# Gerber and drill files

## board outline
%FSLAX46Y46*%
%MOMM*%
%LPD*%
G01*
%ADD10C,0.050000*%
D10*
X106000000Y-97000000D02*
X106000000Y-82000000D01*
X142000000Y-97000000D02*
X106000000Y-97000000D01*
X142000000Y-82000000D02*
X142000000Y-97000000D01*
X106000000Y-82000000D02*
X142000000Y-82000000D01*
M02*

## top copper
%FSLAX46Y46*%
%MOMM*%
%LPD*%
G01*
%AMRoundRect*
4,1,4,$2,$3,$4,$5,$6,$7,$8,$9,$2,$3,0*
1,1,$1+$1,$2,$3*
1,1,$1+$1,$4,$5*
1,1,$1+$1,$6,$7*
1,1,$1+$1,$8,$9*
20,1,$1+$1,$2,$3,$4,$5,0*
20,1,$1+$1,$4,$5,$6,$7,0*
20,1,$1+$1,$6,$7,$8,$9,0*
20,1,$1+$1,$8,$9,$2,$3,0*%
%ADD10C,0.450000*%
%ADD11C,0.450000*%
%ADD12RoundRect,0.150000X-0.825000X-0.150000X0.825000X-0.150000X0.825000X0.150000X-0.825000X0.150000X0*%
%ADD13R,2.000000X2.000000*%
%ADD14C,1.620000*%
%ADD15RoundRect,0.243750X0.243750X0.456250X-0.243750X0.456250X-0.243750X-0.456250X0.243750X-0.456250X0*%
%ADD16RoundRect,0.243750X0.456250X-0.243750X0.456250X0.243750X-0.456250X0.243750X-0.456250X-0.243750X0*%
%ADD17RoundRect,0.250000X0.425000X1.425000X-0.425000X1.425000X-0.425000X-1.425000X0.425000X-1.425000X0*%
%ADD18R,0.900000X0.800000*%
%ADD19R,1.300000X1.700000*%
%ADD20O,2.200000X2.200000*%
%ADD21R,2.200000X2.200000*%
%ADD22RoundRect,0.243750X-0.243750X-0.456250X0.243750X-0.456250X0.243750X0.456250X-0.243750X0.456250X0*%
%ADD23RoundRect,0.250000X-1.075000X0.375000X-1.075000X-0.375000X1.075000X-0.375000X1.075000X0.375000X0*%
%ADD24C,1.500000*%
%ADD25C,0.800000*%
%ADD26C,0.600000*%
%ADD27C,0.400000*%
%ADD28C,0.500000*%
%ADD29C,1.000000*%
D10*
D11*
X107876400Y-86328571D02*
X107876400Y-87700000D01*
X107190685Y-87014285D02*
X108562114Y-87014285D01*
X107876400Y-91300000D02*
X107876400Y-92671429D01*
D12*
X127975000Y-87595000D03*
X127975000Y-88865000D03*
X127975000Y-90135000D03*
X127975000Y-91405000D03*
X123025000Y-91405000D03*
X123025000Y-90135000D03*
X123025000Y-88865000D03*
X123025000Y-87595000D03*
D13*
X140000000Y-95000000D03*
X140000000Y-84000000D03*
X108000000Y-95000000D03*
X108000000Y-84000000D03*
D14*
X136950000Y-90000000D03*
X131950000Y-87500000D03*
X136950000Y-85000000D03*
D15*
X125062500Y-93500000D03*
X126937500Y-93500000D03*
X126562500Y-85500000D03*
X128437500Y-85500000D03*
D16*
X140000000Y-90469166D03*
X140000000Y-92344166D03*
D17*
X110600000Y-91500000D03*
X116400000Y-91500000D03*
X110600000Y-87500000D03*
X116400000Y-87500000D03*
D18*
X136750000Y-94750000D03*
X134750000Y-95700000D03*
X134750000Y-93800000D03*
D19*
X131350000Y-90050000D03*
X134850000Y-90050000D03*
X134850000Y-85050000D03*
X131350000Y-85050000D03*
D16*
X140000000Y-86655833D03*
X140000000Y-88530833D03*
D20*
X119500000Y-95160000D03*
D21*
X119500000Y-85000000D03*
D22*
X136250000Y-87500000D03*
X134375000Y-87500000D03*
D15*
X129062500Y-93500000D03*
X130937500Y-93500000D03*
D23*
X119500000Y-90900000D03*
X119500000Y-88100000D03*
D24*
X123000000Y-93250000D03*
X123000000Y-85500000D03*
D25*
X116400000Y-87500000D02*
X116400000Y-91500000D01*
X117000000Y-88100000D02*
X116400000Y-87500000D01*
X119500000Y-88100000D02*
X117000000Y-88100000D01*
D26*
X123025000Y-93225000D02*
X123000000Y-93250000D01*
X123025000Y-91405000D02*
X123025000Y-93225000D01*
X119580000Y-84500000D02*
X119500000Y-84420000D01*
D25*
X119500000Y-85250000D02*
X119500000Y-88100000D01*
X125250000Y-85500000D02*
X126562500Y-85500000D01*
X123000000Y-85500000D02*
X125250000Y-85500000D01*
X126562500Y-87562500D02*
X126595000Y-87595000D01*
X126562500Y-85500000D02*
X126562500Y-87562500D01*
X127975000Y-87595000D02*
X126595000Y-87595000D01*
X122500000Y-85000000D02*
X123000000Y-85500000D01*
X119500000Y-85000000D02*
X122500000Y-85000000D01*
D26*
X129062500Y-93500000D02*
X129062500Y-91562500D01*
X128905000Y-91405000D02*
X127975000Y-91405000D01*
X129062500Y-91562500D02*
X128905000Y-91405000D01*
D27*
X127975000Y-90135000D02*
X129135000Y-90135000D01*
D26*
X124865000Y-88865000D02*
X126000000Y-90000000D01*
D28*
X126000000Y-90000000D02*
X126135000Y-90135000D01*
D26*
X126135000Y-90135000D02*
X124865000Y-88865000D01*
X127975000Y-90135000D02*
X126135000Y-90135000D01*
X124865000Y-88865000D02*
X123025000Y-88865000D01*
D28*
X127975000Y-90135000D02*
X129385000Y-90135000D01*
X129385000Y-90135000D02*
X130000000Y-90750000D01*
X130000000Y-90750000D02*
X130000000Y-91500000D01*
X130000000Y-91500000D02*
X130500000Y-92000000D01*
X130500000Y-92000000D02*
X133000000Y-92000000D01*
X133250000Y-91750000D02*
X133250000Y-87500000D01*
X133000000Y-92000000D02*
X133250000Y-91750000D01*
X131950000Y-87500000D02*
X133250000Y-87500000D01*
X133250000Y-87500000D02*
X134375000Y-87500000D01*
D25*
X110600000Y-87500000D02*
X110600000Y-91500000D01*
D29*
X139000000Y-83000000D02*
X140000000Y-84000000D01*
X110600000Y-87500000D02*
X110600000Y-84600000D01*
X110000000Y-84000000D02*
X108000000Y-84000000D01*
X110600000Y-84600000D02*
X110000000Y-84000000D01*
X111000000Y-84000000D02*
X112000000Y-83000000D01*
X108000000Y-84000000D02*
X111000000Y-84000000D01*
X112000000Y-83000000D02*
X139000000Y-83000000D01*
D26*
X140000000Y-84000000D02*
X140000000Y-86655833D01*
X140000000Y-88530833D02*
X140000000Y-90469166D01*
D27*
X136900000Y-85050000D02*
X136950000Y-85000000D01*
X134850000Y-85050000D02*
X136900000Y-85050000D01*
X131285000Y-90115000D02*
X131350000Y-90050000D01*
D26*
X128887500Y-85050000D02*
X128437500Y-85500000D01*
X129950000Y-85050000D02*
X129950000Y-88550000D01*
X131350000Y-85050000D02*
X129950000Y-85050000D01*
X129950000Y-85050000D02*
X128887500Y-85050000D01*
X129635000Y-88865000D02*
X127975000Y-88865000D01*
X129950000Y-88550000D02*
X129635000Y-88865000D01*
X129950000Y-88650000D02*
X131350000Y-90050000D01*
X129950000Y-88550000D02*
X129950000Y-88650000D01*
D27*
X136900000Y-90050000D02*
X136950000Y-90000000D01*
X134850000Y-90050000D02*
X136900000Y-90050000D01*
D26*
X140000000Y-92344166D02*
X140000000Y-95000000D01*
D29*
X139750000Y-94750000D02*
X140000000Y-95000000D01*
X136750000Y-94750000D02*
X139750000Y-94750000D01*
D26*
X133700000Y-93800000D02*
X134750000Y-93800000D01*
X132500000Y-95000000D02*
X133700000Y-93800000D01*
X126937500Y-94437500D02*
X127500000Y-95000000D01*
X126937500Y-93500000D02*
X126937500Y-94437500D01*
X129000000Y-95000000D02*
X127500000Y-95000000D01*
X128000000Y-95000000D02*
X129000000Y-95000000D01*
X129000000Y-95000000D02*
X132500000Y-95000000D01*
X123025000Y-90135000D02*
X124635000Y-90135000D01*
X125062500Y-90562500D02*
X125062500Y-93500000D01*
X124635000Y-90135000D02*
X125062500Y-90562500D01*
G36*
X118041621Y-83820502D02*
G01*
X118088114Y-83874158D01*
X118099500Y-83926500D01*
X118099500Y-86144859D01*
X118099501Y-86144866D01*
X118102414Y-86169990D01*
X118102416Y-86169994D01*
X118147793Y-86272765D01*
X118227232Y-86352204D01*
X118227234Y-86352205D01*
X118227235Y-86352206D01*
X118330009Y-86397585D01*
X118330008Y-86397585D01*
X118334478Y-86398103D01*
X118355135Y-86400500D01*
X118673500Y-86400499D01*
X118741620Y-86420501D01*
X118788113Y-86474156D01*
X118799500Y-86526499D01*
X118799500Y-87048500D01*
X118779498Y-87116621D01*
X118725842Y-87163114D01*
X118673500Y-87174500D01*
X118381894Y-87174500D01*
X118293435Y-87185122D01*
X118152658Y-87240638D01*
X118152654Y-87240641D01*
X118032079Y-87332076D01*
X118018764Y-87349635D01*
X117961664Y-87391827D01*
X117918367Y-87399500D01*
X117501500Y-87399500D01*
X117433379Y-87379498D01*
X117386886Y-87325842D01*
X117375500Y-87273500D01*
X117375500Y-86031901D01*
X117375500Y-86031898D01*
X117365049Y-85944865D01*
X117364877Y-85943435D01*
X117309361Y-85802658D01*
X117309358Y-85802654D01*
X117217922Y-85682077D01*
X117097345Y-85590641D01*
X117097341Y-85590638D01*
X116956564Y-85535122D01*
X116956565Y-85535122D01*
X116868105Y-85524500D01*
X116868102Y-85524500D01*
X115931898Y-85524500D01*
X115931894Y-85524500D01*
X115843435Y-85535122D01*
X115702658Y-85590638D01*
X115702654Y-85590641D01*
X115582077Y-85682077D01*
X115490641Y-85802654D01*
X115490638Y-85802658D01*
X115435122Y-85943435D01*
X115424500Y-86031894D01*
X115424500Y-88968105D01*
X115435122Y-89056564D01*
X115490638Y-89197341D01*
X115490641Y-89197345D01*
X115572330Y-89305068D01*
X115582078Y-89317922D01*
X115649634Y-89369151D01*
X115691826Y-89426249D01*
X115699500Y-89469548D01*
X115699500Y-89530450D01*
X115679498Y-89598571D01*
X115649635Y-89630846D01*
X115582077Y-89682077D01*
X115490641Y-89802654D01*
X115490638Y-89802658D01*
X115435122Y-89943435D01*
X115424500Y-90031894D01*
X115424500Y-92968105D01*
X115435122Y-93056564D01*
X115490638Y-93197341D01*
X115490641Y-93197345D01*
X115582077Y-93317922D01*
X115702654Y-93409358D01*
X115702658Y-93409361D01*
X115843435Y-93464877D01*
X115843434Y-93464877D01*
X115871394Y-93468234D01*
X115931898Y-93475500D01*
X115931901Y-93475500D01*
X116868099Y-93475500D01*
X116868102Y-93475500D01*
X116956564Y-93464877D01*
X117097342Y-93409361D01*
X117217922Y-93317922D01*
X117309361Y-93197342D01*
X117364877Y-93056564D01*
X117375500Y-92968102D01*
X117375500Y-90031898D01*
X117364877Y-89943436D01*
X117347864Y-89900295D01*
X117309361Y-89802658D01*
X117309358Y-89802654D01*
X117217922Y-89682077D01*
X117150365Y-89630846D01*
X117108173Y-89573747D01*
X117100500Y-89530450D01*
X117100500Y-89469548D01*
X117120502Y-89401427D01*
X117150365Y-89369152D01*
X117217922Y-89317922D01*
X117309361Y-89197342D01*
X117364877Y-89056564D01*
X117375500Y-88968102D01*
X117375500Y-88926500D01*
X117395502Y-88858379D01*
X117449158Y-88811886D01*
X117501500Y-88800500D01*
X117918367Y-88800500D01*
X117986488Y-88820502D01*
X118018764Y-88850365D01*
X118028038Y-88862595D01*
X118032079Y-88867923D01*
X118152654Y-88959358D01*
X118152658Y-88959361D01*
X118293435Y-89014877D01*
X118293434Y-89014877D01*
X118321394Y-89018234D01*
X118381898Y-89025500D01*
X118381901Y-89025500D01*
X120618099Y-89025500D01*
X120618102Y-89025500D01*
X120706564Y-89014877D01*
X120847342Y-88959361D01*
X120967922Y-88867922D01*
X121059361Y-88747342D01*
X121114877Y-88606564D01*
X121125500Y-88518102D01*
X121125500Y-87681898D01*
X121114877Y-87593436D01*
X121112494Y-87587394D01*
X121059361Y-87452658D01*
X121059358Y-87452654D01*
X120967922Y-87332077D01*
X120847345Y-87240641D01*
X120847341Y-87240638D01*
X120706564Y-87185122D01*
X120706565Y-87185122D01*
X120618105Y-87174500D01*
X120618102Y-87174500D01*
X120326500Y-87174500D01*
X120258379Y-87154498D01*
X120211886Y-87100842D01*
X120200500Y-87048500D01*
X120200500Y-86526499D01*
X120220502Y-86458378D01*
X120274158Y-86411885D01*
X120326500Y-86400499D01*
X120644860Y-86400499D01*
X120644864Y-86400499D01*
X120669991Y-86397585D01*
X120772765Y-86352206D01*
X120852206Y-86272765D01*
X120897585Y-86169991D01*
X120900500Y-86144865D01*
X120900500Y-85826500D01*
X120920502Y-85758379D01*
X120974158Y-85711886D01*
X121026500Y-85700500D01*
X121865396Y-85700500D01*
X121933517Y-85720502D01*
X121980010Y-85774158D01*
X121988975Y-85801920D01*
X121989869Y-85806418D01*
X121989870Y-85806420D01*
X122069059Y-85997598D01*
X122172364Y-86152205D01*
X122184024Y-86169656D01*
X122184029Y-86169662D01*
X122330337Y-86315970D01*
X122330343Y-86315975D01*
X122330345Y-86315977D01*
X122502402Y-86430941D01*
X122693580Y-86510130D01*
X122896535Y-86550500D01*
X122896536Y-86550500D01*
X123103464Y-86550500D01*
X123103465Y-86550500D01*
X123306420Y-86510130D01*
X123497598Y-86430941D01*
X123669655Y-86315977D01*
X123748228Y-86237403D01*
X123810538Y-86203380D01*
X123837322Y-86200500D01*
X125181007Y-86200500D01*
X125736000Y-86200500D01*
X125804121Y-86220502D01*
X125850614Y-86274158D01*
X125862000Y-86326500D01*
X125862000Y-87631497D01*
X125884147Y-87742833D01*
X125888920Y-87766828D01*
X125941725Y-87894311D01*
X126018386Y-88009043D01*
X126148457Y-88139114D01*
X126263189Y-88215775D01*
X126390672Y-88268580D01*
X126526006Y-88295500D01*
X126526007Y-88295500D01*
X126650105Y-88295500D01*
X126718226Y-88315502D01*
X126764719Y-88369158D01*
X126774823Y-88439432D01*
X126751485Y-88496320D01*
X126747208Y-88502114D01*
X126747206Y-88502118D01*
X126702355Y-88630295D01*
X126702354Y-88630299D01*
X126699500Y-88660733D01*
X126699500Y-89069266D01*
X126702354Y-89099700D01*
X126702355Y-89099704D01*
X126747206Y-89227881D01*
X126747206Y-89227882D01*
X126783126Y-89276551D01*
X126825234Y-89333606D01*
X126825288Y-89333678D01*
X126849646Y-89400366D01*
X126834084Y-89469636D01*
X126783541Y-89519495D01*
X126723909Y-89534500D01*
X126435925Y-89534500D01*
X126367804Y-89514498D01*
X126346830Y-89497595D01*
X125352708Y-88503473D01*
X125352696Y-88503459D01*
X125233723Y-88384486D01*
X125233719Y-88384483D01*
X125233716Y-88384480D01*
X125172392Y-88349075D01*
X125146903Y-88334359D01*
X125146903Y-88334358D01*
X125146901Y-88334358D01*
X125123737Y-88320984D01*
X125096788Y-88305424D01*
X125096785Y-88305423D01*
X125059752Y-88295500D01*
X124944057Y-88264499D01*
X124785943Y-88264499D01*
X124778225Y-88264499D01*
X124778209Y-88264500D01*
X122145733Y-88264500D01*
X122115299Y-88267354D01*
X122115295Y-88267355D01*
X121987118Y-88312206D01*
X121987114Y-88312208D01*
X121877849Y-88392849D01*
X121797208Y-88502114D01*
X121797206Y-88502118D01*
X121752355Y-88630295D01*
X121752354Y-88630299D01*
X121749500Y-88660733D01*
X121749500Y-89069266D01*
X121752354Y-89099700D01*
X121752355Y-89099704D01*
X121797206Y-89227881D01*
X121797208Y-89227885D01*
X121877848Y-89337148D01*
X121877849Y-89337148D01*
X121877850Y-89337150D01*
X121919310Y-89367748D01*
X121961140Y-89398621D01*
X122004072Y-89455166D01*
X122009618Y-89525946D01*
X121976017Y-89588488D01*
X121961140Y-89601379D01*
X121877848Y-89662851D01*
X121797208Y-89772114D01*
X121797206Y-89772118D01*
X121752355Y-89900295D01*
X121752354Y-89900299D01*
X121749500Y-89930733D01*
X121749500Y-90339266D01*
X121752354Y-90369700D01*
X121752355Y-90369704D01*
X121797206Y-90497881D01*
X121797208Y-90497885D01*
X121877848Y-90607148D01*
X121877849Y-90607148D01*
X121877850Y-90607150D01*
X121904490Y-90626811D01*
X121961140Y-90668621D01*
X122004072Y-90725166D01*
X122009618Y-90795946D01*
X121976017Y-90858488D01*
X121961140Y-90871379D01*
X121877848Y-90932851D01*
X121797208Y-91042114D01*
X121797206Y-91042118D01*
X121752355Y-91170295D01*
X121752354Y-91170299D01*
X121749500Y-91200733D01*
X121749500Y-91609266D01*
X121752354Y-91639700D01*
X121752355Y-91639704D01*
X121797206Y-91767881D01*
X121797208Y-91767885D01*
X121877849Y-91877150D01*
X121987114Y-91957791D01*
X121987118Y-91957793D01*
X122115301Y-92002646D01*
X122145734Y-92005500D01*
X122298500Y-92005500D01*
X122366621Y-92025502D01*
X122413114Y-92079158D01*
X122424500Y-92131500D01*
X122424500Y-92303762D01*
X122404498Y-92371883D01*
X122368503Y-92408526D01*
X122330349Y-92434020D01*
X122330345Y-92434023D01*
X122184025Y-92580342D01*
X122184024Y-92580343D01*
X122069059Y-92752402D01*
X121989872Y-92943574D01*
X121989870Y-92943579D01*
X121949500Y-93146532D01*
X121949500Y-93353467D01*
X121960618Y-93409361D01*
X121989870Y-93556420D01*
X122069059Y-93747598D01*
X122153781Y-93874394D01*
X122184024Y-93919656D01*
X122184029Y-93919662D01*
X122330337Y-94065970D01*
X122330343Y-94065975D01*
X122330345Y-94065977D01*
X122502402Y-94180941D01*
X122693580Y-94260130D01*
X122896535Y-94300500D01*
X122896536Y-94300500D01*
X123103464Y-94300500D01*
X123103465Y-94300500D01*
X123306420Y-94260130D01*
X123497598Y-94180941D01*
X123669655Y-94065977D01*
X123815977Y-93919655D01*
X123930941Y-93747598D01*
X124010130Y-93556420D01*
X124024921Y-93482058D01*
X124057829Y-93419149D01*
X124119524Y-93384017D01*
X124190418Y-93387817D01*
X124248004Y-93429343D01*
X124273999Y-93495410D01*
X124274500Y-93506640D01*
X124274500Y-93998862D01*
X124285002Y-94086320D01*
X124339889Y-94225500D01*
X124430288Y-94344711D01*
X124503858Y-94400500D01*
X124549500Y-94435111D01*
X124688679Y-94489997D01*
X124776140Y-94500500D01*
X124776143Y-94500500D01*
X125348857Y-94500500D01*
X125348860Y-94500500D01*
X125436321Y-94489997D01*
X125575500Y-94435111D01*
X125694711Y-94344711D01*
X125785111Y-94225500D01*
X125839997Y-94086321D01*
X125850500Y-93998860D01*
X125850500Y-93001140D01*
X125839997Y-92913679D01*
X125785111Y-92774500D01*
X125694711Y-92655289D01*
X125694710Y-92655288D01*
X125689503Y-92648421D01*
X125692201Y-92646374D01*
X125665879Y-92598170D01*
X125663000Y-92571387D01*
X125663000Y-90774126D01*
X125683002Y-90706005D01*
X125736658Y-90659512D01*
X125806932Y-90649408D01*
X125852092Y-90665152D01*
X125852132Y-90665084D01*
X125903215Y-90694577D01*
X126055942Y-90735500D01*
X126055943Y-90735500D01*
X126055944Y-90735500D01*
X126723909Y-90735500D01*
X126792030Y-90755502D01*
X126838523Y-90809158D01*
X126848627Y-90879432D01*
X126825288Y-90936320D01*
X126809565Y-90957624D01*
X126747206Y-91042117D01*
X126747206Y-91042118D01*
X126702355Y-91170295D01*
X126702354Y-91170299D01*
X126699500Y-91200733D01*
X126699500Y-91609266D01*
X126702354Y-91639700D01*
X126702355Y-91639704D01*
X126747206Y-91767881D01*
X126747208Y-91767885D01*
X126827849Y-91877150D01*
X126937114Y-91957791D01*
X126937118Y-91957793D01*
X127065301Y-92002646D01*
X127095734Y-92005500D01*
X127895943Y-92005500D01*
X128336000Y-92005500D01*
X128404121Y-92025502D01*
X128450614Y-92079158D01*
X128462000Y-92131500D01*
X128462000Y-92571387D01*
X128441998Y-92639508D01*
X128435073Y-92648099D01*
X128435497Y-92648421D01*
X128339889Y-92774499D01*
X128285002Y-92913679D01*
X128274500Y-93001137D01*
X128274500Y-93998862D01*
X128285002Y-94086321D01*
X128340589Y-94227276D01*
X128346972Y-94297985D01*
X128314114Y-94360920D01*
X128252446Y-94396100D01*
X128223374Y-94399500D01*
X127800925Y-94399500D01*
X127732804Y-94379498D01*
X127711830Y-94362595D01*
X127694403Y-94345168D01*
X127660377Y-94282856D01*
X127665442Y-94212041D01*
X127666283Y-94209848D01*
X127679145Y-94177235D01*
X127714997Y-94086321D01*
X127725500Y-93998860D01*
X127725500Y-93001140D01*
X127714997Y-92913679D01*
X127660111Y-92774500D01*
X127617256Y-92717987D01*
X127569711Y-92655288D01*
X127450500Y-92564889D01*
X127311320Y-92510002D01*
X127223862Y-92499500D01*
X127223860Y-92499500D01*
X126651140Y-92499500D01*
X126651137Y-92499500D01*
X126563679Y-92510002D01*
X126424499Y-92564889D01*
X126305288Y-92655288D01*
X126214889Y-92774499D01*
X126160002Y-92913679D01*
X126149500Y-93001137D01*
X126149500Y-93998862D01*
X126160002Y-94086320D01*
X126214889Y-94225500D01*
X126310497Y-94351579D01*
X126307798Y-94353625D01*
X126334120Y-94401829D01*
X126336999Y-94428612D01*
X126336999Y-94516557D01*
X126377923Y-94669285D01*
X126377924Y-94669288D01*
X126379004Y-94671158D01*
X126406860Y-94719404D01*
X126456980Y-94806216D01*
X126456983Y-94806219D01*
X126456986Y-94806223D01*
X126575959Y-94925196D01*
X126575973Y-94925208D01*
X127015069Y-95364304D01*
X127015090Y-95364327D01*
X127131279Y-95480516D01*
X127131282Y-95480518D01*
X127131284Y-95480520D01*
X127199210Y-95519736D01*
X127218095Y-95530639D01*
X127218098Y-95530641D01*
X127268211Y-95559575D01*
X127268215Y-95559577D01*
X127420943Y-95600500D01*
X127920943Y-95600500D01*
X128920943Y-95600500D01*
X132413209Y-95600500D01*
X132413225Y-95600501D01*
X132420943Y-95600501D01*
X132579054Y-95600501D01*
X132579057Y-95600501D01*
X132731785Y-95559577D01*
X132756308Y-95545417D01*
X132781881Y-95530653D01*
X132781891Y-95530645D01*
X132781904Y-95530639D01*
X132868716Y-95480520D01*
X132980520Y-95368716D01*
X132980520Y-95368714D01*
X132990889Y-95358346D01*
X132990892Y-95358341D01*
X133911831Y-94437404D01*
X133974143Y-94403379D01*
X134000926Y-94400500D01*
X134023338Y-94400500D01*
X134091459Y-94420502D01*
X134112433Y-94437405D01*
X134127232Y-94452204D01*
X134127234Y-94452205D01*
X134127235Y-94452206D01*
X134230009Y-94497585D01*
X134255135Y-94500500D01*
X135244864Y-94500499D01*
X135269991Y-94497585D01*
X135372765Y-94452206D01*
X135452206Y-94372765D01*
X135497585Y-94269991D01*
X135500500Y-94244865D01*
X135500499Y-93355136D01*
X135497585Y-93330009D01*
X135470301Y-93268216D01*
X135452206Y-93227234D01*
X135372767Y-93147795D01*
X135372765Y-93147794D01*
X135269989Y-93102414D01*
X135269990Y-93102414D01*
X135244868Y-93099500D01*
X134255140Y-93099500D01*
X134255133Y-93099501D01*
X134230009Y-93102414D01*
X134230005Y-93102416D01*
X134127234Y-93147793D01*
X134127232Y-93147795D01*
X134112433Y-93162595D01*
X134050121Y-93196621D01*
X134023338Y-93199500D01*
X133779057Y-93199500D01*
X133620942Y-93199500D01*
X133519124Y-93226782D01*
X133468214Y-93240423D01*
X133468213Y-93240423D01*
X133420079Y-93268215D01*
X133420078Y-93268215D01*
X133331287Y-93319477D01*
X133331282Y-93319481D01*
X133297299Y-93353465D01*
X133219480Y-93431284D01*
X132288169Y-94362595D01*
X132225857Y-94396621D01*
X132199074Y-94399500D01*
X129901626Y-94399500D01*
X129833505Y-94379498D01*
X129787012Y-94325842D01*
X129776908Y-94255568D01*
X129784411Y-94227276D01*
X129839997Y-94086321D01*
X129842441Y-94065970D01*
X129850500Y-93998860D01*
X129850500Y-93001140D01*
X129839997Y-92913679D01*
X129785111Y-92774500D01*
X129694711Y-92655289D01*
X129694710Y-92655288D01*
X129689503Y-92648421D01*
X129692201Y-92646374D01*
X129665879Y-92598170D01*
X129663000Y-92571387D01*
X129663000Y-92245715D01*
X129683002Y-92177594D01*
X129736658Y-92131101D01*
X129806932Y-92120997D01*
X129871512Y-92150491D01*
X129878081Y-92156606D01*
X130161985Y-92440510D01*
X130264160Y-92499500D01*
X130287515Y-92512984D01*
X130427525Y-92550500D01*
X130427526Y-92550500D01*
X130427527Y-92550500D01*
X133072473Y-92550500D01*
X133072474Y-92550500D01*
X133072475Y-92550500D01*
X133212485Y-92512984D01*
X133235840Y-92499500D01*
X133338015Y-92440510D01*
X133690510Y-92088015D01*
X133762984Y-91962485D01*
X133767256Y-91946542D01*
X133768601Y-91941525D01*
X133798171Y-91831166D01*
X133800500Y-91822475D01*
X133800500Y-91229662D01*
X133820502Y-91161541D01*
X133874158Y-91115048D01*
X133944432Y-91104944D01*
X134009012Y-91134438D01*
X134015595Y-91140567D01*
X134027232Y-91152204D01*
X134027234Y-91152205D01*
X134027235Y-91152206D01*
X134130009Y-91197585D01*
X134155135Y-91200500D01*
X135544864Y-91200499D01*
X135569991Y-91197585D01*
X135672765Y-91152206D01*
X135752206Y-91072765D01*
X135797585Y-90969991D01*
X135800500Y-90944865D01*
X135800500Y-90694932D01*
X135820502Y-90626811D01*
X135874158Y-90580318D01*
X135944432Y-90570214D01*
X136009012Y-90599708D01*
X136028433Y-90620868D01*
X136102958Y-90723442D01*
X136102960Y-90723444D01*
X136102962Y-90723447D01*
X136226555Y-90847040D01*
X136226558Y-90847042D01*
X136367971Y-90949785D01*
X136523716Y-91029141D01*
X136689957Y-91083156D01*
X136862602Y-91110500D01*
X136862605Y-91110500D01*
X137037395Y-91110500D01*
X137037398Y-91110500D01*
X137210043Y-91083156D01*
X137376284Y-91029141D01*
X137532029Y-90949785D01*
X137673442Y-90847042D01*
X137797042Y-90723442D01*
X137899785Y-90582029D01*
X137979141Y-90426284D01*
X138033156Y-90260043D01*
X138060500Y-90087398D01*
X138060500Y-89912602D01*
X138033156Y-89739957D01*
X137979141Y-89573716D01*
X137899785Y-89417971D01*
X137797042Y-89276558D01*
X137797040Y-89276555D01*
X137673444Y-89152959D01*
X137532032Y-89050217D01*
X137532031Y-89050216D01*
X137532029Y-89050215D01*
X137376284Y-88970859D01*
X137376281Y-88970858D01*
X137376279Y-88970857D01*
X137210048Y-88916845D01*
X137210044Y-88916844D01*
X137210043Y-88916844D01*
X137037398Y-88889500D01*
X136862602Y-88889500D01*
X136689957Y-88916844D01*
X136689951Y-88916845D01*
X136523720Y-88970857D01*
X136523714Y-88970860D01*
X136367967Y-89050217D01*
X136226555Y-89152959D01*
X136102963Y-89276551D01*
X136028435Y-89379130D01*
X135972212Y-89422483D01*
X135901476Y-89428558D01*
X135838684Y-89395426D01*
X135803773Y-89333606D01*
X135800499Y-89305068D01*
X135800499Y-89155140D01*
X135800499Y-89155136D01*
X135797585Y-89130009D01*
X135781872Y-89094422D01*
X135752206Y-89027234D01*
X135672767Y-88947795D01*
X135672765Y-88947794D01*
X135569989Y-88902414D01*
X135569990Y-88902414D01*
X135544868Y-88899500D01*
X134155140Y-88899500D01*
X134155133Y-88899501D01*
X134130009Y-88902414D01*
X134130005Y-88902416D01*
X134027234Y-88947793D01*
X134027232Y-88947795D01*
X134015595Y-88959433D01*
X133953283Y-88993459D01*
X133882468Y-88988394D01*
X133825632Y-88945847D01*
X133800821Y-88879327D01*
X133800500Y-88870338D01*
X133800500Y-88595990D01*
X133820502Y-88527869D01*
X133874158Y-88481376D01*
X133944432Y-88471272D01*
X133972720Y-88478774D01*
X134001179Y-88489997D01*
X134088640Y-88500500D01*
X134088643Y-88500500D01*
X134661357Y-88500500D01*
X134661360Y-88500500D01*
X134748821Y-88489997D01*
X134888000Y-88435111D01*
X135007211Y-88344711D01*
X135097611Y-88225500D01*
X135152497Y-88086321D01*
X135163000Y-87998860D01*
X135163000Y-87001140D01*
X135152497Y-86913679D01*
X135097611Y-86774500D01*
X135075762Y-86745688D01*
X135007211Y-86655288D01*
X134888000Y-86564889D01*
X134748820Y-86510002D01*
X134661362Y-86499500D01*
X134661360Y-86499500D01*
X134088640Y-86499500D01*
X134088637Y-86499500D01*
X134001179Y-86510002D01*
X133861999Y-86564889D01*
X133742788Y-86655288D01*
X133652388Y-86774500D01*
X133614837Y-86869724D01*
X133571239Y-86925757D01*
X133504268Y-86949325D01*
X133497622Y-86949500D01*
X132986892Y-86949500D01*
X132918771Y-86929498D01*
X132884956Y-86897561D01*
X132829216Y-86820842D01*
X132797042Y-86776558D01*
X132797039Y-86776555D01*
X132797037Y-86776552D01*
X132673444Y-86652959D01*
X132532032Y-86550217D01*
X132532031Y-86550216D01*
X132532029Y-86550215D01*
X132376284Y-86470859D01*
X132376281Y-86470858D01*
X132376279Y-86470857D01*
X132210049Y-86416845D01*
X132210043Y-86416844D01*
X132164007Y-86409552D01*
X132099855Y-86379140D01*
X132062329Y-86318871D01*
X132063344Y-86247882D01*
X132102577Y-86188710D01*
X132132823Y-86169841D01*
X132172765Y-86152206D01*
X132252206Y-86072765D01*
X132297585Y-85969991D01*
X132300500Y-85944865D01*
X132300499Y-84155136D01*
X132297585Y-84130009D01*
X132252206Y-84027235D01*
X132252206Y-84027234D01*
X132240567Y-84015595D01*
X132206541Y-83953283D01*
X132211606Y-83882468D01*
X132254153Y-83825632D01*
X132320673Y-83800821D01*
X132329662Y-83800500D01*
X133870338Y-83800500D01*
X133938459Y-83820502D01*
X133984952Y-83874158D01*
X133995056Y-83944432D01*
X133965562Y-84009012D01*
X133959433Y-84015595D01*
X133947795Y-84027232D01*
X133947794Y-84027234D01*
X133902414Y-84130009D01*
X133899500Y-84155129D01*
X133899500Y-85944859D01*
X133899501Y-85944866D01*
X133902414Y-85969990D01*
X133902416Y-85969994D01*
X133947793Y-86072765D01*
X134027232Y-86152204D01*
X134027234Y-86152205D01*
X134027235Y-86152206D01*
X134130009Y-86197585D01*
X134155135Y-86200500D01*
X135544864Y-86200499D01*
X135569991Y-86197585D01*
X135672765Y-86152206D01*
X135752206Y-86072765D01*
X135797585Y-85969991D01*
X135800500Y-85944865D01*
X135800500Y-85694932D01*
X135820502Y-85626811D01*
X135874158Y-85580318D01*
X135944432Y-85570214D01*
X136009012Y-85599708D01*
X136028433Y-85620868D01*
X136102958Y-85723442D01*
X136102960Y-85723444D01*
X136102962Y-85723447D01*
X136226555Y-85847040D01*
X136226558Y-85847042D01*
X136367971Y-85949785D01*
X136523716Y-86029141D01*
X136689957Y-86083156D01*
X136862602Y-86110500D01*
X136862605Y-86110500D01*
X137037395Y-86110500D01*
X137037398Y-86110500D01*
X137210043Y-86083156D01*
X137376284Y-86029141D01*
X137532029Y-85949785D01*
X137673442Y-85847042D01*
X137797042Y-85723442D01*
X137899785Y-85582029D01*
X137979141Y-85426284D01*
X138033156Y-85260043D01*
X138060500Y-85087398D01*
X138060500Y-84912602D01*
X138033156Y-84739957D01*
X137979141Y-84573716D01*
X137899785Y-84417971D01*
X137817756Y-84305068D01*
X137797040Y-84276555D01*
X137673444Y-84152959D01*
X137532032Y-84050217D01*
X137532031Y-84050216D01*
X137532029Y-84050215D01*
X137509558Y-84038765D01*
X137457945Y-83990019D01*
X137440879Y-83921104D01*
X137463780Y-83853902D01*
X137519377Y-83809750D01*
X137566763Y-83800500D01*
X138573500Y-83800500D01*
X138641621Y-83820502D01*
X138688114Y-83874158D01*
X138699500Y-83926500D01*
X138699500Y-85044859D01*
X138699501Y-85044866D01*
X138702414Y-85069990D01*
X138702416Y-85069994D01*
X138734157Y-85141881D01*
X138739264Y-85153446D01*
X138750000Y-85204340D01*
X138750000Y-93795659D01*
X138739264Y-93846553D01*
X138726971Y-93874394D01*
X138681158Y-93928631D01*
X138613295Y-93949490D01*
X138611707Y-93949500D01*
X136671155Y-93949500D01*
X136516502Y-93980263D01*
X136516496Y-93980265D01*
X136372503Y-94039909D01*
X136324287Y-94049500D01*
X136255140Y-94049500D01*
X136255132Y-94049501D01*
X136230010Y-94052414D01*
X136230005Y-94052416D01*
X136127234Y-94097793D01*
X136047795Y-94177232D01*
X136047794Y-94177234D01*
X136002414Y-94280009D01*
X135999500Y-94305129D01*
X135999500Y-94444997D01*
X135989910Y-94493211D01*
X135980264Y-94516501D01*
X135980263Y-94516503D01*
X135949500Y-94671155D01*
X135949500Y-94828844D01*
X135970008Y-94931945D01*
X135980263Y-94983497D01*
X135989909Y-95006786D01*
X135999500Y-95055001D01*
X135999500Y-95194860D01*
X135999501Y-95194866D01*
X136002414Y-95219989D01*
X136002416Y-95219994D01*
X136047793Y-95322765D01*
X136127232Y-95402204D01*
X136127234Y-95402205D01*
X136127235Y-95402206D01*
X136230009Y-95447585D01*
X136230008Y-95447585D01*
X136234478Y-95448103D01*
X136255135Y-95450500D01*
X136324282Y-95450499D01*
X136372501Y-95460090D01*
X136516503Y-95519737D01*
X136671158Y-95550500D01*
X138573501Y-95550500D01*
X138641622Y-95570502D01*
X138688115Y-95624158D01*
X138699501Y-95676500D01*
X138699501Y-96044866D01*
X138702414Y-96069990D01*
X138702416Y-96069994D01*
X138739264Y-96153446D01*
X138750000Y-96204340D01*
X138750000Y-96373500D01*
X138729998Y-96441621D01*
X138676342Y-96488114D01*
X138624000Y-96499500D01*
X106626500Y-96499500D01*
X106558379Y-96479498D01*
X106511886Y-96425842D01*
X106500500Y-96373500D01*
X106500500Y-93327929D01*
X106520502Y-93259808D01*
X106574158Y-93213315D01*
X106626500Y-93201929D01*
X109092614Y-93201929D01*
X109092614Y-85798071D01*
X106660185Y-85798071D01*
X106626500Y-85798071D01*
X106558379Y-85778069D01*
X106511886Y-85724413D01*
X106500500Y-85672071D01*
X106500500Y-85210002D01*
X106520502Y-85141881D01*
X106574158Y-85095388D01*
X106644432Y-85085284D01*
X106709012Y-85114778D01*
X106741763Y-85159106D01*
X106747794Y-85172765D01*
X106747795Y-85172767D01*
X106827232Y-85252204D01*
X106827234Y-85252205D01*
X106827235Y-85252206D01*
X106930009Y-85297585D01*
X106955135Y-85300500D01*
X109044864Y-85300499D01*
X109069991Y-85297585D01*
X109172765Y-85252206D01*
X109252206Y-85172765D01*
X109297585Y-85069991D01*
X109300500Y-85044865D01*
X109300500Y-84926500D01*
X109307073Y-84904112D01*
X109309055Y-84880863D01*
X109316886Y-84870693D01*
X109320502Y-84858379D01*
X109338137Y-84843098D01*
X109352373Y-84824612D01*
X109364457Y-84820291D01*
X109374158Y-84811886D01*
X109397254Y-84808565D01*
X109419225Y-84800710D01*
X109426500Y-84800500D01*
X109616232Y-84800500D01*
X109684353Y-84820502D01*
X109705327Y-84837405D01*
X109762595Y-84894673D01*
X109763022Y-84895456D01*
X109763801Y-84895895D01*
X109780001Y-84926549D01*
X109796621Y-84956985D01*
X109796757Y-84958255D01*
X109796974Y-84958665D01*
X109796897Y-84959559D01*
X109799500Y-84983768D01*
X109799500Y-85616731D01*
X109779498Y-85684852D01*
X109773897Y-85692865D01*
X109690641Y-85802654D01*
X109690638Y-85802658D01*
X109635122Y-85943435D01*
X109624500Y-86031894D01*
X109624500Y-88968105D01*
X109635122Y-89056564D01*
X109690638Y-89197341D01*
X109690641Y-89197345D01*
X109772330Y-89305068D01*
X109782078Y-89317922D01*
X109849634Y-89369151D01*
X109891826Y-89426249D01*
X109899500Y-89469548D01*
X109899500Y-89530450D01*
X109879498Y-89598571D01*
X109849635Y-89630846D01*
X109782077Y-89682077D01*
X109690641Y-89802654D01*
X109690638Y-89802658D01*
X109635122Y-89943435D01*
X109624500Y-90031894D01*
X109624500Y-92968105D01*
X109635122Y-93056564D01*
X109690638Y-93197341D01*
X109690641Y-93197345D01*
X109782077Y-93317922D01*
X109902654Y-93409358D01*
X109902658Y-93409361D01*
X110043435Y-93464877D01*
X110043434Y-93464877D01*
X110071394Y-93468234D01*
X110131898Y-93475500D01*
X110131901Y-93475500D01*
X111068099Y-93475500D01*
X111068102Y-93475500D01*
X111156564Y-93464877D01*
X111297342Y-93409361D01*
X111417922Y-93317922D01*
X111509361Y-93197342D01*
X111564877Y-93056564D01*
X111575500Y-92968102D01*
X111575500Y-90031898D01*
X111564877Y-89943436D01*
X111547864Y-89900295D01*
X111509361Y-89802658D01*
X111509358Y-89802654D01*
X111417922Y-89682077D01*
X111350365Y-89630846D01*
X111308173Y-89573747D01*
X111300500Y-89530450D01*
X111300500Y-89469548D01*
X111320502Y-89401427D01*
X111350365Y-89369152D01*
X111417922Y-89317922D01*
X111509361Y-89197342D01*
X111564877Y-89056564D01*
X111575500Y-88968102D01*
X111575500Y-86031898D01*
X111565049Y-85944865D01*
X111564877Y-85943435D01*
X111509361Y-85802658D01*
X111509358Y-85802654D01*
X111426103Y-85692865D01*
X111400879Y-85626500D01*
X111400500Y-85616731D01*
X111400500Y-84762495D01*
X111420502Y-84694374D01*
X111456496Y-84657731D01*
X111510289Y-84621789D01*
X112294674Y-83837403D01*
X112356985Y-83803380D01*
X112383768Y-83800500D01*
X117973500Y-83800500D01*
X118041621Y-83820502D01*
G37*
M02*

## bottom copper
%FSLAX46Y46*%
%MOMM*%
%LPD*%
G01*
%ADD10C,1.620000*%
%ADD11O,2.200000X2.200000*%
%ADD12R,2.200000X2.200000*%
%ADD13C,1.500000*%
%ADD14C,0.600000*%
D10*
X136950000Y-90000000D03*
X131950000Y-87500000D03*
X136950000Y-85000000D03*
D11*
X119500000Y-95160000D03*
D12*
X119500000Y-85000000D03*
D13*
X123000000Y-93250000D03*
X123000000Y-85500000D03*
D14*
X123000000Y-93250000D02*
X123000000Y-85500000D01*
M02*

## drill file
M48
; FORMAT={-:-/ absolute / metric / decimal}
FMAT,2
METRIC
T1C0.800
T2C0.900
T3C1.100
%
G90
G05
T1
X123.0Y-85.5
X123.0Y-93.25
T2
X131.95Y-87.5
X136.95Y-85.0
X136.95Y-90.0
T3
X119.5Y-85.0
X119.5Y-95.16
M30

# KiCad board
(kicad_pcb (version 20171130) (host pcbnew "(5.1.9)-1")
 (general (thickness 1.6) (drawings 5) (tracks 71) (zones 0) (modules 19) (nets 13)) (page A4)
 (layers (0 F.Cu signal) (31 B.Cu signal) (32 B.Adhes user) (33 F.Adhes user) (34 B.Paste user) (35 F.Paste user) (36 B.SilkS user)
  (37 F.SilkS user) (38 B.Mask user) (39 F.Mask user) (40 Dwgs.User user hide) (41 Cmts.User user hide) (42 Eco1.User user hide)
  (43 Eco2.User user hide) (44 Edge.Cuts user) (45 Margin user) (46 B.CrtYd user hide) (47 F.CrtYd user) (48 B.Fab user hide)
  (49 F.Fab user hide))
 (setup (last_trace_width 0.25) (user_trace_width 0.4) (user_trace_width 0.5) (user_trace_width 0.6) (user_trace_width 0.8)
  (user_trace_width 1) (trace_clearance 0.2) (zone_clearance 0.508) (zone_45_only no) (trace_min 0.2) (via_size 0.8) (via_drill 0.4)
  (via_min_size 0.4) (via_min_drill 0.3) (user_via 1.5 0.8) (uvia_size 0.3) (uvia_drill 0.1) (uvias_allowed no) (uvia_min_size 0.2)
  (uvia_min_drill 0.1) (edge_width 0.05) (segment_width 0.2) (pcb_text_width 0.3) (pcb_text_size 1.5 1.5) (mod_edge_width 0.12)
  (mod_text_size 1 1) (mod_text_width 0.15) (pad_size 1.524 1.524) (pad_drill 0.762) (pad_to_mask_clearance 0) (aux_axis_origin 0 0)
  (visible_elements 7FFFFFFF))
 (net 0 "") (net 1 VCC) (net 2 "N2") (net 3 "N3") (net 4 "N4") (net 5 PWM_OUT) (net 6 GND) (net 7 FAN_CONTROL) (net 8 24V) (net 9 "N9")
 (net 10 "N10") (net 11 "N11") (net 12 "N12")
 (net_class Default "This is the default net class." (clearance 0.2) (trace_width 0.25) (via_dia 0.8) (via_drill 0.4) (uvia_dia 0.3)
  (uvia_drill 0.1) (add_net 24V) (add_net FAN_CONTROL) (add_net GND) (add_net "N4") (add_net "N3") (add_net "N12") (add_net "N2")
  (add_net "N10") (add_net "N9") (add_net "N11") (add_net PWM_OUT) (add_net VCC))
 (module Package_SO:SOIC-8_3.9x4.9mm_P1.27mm (layer F.Cu) (at 125.5 89.5)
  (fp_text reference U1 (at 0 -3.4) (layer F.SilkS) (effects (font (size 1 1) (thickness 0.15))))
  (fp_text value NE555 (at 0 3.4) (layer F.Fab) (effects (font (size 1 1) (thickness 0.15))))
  (pad 8 smd roundrect (at 2.475 -1.905) (size 1.95 0.6) (layers F.Cu F.Paste F.Mask) (roundrect_rratio 0.25) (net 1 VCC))
  (pad 7 smd roundrect (at 2.475 -0.635) (size 1.95 0.6) (layers F.Cu F.Paste F.Mask) (roundrect_rratio 0.25) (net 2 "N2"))
  (pad 6 smd roundrect (at 2.475 0.635) (size 1.95 0.6) (layers F.Cu F.Paste F.Mask) (roundrect_rratio 0.25) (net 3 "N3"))
  (pad 5 smd roundrect (at 2.475 1.905) (size 1.95 0.6) (layers F.Cu F.Paste F.Mask) (roundrect_rratio 0.25) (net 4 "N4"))
  (pad 4 smd roundrect (at -2.475 1.905) (size 1.95 0.6) (layers F.Cu F.Paste F.Mask) (roundrect_rratio 0.25) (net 1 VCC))
  (pad 3 smd roundrect (at -2.475 0.635) (size 1.95 0.6) (layers F.Cu F.Paste F.Mask) (roundrect_rratio 0.25) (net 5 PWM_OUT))
  (pad 2 smd roundrect (at -2.475 -0.635) (size 1.95 0.6) (layers F.Cu F.Paste F.Mask) (roundrect_rratio 0.25) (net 3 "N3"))
  (pad 1 smd roundrect (at -2.475 -1.905) (size 1.95 0.6) (layers F.Cu F.Paste F.Mask) (roundrect_rratio 0.25) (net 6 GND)))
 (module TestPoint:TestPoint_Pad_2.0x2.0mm (layer F.Cu) (at 140 95)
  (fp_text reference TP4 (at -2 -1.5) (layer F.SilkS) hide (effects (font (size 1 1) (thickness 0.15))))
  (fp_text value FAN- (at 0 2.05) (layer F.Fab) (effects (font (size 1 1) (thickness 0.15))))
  (pad 1 smd rect (at 0 0) (size 2 2) (layers F.Cu F.Mask) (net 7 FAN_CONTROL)))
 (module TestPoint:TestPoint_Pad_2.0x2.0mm (layer F.Cu) (at 140 84)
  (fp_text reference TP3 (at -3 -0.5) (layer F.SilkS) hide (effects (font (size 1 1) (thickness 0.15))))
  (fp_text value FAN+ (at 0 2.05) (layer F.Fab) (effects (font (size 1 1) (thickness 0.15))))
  (pad 1 smd rect (at 0 0) (size 2 2) (layers F.Cu F.Mask) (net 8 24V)))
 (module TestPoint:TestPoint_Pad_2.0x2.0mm (layer F.Cu) (at 108 95)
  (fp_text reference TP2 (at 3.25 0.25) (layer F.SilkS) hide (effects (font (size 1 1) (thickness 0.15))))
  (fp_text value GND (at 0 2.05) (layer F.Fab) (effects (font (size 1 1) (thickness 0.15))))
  (pad 1 smd rect (at 0 0) (size 2 2) (layers F.Cu F.Mask) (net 6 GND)))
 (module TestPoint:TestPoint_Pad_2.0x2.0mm (layer F.Cu) (at 108 84)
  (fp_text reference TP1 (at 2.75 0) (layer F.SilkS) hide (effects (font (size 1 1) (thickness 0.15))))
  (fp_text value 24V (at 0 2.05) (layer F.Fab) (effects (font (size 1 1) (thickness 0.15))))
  (pad 1 smd rect (at 0 0) (size 2 2) (layers F.Cu F.Mask) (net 8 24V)))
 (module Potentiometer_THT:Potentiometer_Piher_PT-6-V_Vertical (layer B.Cu) (at 136.95 90 180)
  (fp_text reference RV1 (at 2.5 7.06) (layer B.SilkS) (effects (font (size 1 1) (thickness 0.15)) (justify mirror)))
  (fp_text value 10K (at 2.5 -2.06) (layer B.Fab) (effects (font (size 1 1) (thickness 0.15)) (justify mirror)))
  (pad 1 thru_hole circle (at 0 0 180) (size 1.62 1.62) (drill 0.9) (layers *.Cu *.Mask) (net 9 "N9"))
  (pad 2 thru_hole circle (at 5 2.5 180) (size 1.62 1.62) (drill 0.9) (layers *.Cu *.Mask) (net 3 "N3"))
  (pad 3 thru_hole circle (at 0 5 180) (size 1.62 1.62) (drill 0.9) (layers *.Cu *.Mask) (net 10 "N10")))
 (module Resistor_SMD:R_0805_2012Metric (layer F.Cu) (at 126 93.5 180)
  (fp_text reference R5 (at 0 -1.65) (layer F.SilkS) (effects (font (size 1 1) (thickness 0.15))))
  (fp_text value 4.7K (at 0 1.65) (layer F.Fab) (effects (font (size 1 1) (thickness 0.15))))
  (pad 2 smd roundrect (at 0.9375 0 180) (size 0.975 1.4) (layers F.Cu F.Paste F.Mask) (roundrect_rratio 0.25) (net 5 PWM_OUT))
  (pad 1 smd roundrect (at -0.9375 0 180) (size 0.975 1.4) (layers F.Cu F.Paste F.Mask) (roundrect_rratio 0.25) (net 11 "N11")))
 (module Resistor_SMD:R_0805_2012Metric (layer F.Cu) (at 127.5 85.5 180)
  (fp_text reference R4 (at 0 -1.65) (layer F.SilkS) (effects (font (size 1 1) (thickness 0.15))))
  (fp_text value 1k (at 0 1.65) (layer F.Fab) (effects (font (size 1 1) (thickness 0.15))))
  (pad 2 smd roundrect (at 0.9375 0 180) (size 0.975 1.4) (layers F.Cu F.Paste F.Mask) (roundrect_rratio 0.25) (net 1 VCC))
  (pad 1 smd roundrect (at -0.9375 0 180) (size 0.975 1.4) (layers F.Cu F.Paste F.Mask) (roundrect_rratio 0.25) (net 2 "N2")))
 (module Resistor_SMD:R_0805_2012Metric (layer F.Cu) (at 140 91.406666 90)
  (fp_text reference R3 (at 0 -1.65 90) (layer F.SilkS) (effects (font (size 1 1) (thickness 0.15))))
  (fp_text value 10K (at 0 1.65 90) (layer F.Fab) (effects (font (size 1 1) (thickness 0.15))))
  (pad 2 smd roundrect (at 0.9375 0 90) (size 0.975 1.4) (layers F.Cu F.Paste F.Mask) (roundrect_rratio 0.25) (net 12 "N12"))
  (pad 1 smd roundrect (at -0.9375 0 90) (size 0.975 1.4) (layers F.Cu F.Paste F.Mask) (roundrect_rratio 0.25) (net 7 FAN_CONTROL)))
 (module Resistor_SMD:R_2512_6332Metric (layer F.Cu) (at 113.5 91.5 180)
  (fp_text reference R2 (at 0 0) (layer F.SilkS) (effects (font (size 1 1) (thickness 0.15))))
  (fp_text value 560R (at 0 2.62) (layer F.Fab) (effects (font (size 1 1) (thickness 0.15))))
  (pad 2 smd roundrect (at 2.9 0 180) (size 1.35 3.35) (layers F.Cu F.Paste F.Mask) (roundrect_rratio 0.185185) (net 8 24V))
  (pad 1 smd roundrect (at -2.9 0 180) (size 1.35 3.35) (layers F.Cu F.Paste F.Mask) (roundrect_rratio 0.185185) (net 1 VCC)))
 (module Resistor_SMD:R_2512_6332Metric (layer F.Cu) (at 113.5 87.5 180)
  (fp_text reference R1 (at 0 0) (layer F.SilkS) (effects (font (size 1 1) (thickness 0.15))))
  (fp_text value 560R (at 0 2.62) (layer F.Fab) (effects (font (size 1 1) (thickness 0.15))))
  (pad 2 smd roundrect (at 2.9 0 180) (size 1.35 3.35) (layers F.Cu F.Paste F.Mask) (roundrect_rratio 0.185185) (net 8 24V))
  (pad 1 smd roundrect (at -2.9 0 180) (size 1.35 3.35) (layers F.Cu F.Paste F.Mask) (roundrect_rratio 0.185185) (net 1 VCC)))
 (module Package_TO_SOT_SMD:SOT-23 (layer F.Cu) (at 135.75 94.75)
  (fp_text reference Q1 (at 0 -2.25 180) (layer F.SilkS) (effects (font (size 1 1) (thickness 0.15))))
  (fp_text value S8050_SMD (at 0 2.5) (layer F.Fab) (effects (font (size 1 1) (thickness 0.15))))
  (pad 3 smd rect (at 1 0) (size 0.9 0.8) (layers F.Cu F.Paste F.Mask) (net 7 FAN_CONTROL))
  (pad 2 smd rect (at -1 0.95) (size 0.9 0.8) (layers F.Cu F.Paste F.Mask) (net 6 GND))
  (pad 1 smd rect (at -1 -0.95) (size 0.9 0.8) (layers F.Cu F.Paste F.Mask) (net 11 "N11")))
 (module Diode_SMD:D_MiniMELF (layer F.Cu) (at 133.1 90.05 180)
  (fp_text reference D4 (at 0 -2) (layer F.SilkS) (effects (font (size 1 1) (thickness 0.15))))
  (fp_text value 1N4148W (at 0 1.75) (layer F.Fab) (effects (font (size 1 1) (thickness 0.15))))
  (pad 2 smd rect (at 1.75 0 180) (size 1.3 1.7) (layers F.Cu F.Paste F.Mask) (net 2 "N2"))
  (pad 1 smd rect (at -1.75 0 180) (size 1.3 1.7) (layers F.Cu F.Paste F.Mask) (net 9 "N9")))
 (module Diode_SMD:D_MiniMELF (layer F.Cu) (at 133.1 85.05)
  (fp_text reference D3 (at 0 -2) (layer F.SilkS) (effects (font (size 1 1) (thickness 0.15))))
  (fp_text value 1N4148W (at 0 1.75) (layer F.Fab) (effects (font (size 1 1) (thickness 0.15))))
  (pad 2 smd rect (at 1.75 0) (size 1.3 1.7) (layers F.Cu F.Paste F.Mask) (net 10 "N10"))
  (pad 1 smd rect (at -1.75 0) (size 1.3 1.7) (layers F.Cu F.Paste F.Mask) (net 2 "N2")))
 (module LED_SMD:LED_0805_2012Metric (layer F.Cu) (at 140 87.593333 90)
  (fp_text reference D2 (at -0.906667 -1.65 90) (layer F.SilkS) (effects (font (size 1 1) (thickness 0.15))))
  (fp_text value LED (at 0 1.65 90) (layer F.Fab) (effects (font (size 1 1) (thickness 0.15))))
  (pad 2 smd roundrect (at 0.9375 0 90) (size 0.975 1.4) (layers F.Cu F.Paste F.Mask) (roundrect_rratio 0.25) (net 8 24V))
  (pad 1 smd roundrect (at -0.9375 0 90) (size 0.975 1.4) (layers F.Cu F.Paste F.Mask) (roundrect_rratio 0.25) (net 12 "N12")))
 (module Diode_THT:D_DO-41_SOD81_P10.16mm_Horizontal (layer B.Cu) (at 119.5 85 270)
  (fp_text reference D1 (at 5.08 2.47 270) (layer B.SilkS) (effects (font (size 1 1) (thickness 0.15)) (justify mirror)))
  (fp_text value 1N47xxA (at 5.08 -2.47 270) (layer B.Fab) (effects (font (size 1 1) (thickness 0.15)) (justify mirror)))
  (pad 2 thru_hole oval (at 10.16 0 270) (size 2.2 2.2) (drill 1.1) (layers *.Cu *.Mask) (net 6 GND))
  (pad 1 thru_hole rect (at 0 0 270) (size 2.2 2.2) (drill 1.1) (layers *.Cu *.Mask) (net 1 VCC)))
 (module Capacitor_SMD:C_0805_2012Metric (layer F.Cu) (at 135.3125 87.5)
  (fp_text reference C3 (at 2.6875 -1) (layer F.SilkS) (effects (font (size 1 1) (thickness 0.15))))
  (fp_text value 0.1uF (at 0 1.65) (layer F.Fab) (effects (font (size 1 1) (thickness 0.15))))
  (pad 2 smd roundrect (at 0.9375 0) (size 0.975 1.4) (layers F.Cu F.Paste F.Mask) (roundrect_rratio 0.25) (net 6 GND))
  (pad 1 smd roundrect (at -0.9375 0) (size 0.975 1.4) (layers F.Cu F.Paste F.Mask) (roundrect_rratio 0.25) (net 3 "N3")))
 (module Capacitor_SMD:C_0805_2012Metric (layer F.Cu) (at 130 93.5 180)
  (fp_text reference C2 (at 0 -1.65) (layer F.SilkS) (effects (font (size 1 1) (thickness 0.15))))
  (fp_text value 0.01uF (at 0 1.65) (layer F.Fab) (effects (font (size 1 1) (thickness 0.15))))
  (pad 2 smd roundrect (at 0.9375 0 180) (size 0.975 1.4) (layers F.Cu F.Paste F.Mask) (roundrect_rratio 0.25) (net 4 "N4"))
  (pad 1 smd roundrect (at -0.9375 0 180) (size 0.975 1.4) (layers F.Cu F.Paste F.Mask) (roundrect_rratio 0.25) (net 6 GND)))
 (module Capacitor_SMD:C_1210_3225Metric (layer F.Cu) (at 119.5 89.5 270)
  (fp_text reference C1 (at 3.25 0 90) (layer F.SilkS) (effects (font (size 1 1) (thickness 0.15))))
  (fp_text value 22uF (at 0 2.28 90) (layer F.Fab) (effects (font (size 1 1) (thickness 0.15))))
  (pad 2 smd roundrect (at 1.4 0 270) (size 1.25 2.65) (layers F.Cu F.Paste F.Mask) (roundrect_rratio 0.2) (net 6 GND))
  (pad 1 smd roundrect (at -1.4 0 270) (size 1.25 2.65) (layers F.Cu F.Paste F.Mask) (roundrect_rratio 0.2) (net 1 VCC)))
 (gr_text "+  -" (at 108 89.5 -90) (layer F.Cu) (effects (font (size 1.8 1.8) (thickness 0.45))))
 (gr_line (start 106 97) (end 106 82) (layer Edge.Cuts) (width 0.05))
 (gr_line (start 142 97) (end 106 97) (layer Edge.Cuts) (width 0.05))
 (gr_line (start 142 82) (end 142 97) (layer Edge.Cuts) (width 0.05))
 (gr_line (start 106 82) (end 142 82) (layer Edge.Cuts) (width 0.05))
 (segment (start 116.4 87.5) (end 116.4 91.5) (width 0.8) (layer F.Cu) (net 1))
 (segment (start 117 88.1) (end 116.4 87.5) (width 0.8) (layer F.Cu) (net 1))
 (segment (start 119.5 88.1) (end 117 88.1) (width 0.8) (layer F.Cu) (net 1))
 (via (at 123 93.25) (size 1.5) (drill 0.8) (layers F.Cu B.Cu) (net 1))
 (segment (start 123.025 93.225) (end 123 93.25) (width 0.6) (layer F.Cu) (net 1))
 (segment (start 123.025 91.405) (end 123.025 93.225) (width 0.6) (layer F.Cu) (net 1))
 (via (at 123 85.5) (size 1.5) (drill 0.8) (layers F.Cu B.Cu) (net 1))
 (segment (start 123 93.25) (end 123 85.5) (width 0.6) (layer B.Cu) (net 1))
 (segment (start 119.58 84.5) (end 119.5 84.42) (width 0.6) (layer F.Cu) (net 1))
 (segment (start 119.5 85.25) (end 119.5 88.1) (width 0.8) (layer F.Cu) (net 1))
 (segment (start 125.25 85.5) (end 126.5625 85.5) (width 0.8) (layer F.Cu) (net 1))
 (segment (start 123 85.5) (end 125.25 85.5) (width 0.8) (layer F.Cu) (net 1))
 (segment (start 126.5625 87.5625) (end 126.595 87.595) (width 0.8) (layer F.Cu) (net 1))
 (segment (start 126.5625 85.5) (end 126.5625 87.5625) (width 0.8) (layer F.Cu) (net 1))
 (segment (start 127.975 87.595) (end 126.595 87.595) (width 0.8) (layer F.Cu) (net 1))
 (segment (start 122.5 85) (end 123 85.5) (width 0.8) (layer F.Cu) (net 1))
 (segment (start 119.5 85) (end 122.5 85) (width 0.8) (layer F.Cu) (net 1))
 (segment (start 129.0625 93.5) (end 129.0625 91.5625) (width 0.6) (layer F.Cu) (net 4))
 (segment (start 128.905 91.405) (end 127.975 91.405) (width 0.6) (layer F.Cu) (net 4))
 (segment (start 129.0625 91.5625) (end 128.905 91.405) (width 0.6) (layer F.Cu) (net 4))
 (segment (start 127.975 90.135) (end 129.135 90.135) (width 0.4) (layer F.Cu) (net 3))
 (segment (start 124.865 88.865) (end 126 90) (width 0.6) (layer F.Cu) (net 3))
 (segment (start 126 90) (end 126.135 90.135) (width 0.5) (layer F.Cu) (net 3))
 (segment (start 126.135 90.135) (end 124.865 88.865) (width 0.6) (layer F.Cu) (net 3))
 (segment (start 127.975 90.135) (end 126.135 90.135) (width 0.6) (layer F.Cu) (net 3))
 (segment (start 124.865 88.865) (end 123.025 88.865) (width 0.6) (layer F.Cu) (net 3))
 (segment (start 127.975 90.135) (end 129.385 90.135) (width 0.5) (layer F.Cu) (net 3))
 (segment (start 129.385 90.135) (end 130 90.75) (width 0.5) (layer F.Cu) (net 3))
 (segment (start 130 90.75) (end 130 91.5) (width 0.5) (layer F.Cu) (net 3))
 (segment (start 130 91.5) (end 130.5 92) (width 0.5) (layer F.Cu) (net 3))
 (segment (start 130.5 92) (end 133 92) (width 0.5) (layer F.Cu) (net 3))
 (segment (start 133.25 91.75) (end 133.25 87.5) (width 0.5) (layer F.Cu) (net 3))
 (segment (start 133 92) (end 133.25 91.75) (width 0.5) (layer F.Cu) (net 3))
 (segment (start 131.95 87.5) (end 133.25 87.5) (width 0.5) (layer F.Cu) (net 3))
 (segment (start 133.25 87.5) (end 134.375 87.5) (width 0.5) (layer F.Cu) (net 3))
 (segment (start 110.6 87.5) (end 110.6 91.5) (width 0.8) (layer F.Cu) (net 8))
 (segment (start 139 83) (end 140 84) (width 1) (layer F.Cu) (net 8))
 (segment (start 110.6 87.5) (end 110.6 84.6) (width 1) (layer F.Cu) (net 8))
 (segment (start 110 84) (end 108 84) (width 1) (layer F.Cu) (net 8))
 (segment (start 110.6 84.6) (end 110 84) (width 1) (layer F.Cu) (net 8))
 (segment (start 111 84) (end 112 83) (width 1) (layer F.Cu) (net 8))
 (segment (start 108 84) (end 111 84) (width 1) (layer F.Cu) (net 8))
 (segment (start 112 83) (end 139 83) (width 1) (layer F.Cu) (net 8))
 (segment (start 140 84) (end 140 86.655833) (width 0.6) (layer F.Cu) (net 8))
 (segment (start 140 88.530833) (end 140 90.469166) (width 0.6) (layer F.Cu) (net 12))
 (segment (start 136.9 85.05) (end 136.95 85) (width 0.4) (layer F.Cu) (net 10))
 (segment (start 134.85 85.05) (end 136.9 85.05) (width 0.4) (layer F.Cu) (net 10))
 (segment (start 131.285 90.115) (end 131.35 90.05) (width 0.4) (layer F.Cu) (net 2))
 (segment (start 128.8875 85.05) (end 128.4375 85.5) (width 0.6) (layer F.Cu) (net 2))
 (segment (start 129.95 85.05) (end 129.95 88.55) (width 0.6) (layer F.Cu) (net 2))
 (segment (start 131.35 85.05) (end 129.95 85.05) (width 0.6) (layer F.Cu) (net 2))
 (segment (start 129.95 85.05) (end 128.8875 85.05) (width 0.6) (layer F.Cu) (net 2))
 (segment (start 129.635 88.865) (end 127.975 88.865) (width 0.6) (layer F.Cu) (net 2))
 (segment (start 129.95 88.55) (end 129.635 88.865) (width 0.6) (layer F.Cu) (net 2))
 (segment (start 129.95 88.65) (end 131.35 90.05) (width 0.6) (layer F.Cu) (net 2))
 (segment (start 129.95 88.55) (end 129.95 88.65) (width 0.6) (layer F.Cu) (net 2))
 (segment (start 136.9 90.05) (end 136.95 90) (width 0.4) (layer F.Cu) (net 9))
 (segment (start 134.85 90.05) (end 136.9 90.05) (width 0.4) (layer F.Cu) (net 9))
 (segment (start 140 92.344166) (end 140 95) (width 0.6) (layer F.Cu) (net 7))
 (segment (start 139.75 94.75) (end 140 95) (width 1) (layer F.Cu) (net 7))
 (segment (start 136.75 94.75) (end 139.75 94.75) (width 1) (layer F.Cu) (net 7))
 (segment (start 133.7 93.8) (end 134.75 93.8) (width 0.6) (layer F.Cu) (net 11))
 (segment (start 132.5 95) (end 133.7 93.8) (width 0.6) (layer F.Cu) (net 11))
 (segment (start 126.9375 94.4375) (end 127.5 95) (width 0.6) (layer F.Cu) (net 11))
 (segment (start 126.9375 93.5) (end 126.9375 94.4375) (width 0.6) (layer F.Cu) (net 11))
 (segment (start 129 95) (end 127.5 95) (width 0.6) (layer F.Cu) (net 11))
 (segment (start 128 95) (end 129 95) (width 0.6) (layer F.Cu) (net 11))
 (segment (start 129 95) (end 132.5 95) (width 0.6) (layer F.Cu) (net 11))
 (segment (start 123.025 90.135) (end 124.635 90.135) (width 0.6) (layer F.Cu) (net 5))
 (segment (start 125.0625 90.5625) (end 125.0625 93.5) (width 0.6) (layer F.Cu) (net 5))
 (segment (start 124.635 90.135) (end 125.0625 90.5625) (width 0.6) (layer F.Cu) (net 5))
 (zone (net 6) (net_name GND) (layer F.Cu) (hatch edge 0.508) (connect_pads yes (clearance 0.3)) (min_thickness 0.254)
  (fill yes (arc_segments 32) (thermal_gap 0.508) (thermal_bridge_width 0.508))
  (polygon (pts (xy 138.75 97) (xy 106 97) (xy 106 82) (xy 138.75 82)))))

